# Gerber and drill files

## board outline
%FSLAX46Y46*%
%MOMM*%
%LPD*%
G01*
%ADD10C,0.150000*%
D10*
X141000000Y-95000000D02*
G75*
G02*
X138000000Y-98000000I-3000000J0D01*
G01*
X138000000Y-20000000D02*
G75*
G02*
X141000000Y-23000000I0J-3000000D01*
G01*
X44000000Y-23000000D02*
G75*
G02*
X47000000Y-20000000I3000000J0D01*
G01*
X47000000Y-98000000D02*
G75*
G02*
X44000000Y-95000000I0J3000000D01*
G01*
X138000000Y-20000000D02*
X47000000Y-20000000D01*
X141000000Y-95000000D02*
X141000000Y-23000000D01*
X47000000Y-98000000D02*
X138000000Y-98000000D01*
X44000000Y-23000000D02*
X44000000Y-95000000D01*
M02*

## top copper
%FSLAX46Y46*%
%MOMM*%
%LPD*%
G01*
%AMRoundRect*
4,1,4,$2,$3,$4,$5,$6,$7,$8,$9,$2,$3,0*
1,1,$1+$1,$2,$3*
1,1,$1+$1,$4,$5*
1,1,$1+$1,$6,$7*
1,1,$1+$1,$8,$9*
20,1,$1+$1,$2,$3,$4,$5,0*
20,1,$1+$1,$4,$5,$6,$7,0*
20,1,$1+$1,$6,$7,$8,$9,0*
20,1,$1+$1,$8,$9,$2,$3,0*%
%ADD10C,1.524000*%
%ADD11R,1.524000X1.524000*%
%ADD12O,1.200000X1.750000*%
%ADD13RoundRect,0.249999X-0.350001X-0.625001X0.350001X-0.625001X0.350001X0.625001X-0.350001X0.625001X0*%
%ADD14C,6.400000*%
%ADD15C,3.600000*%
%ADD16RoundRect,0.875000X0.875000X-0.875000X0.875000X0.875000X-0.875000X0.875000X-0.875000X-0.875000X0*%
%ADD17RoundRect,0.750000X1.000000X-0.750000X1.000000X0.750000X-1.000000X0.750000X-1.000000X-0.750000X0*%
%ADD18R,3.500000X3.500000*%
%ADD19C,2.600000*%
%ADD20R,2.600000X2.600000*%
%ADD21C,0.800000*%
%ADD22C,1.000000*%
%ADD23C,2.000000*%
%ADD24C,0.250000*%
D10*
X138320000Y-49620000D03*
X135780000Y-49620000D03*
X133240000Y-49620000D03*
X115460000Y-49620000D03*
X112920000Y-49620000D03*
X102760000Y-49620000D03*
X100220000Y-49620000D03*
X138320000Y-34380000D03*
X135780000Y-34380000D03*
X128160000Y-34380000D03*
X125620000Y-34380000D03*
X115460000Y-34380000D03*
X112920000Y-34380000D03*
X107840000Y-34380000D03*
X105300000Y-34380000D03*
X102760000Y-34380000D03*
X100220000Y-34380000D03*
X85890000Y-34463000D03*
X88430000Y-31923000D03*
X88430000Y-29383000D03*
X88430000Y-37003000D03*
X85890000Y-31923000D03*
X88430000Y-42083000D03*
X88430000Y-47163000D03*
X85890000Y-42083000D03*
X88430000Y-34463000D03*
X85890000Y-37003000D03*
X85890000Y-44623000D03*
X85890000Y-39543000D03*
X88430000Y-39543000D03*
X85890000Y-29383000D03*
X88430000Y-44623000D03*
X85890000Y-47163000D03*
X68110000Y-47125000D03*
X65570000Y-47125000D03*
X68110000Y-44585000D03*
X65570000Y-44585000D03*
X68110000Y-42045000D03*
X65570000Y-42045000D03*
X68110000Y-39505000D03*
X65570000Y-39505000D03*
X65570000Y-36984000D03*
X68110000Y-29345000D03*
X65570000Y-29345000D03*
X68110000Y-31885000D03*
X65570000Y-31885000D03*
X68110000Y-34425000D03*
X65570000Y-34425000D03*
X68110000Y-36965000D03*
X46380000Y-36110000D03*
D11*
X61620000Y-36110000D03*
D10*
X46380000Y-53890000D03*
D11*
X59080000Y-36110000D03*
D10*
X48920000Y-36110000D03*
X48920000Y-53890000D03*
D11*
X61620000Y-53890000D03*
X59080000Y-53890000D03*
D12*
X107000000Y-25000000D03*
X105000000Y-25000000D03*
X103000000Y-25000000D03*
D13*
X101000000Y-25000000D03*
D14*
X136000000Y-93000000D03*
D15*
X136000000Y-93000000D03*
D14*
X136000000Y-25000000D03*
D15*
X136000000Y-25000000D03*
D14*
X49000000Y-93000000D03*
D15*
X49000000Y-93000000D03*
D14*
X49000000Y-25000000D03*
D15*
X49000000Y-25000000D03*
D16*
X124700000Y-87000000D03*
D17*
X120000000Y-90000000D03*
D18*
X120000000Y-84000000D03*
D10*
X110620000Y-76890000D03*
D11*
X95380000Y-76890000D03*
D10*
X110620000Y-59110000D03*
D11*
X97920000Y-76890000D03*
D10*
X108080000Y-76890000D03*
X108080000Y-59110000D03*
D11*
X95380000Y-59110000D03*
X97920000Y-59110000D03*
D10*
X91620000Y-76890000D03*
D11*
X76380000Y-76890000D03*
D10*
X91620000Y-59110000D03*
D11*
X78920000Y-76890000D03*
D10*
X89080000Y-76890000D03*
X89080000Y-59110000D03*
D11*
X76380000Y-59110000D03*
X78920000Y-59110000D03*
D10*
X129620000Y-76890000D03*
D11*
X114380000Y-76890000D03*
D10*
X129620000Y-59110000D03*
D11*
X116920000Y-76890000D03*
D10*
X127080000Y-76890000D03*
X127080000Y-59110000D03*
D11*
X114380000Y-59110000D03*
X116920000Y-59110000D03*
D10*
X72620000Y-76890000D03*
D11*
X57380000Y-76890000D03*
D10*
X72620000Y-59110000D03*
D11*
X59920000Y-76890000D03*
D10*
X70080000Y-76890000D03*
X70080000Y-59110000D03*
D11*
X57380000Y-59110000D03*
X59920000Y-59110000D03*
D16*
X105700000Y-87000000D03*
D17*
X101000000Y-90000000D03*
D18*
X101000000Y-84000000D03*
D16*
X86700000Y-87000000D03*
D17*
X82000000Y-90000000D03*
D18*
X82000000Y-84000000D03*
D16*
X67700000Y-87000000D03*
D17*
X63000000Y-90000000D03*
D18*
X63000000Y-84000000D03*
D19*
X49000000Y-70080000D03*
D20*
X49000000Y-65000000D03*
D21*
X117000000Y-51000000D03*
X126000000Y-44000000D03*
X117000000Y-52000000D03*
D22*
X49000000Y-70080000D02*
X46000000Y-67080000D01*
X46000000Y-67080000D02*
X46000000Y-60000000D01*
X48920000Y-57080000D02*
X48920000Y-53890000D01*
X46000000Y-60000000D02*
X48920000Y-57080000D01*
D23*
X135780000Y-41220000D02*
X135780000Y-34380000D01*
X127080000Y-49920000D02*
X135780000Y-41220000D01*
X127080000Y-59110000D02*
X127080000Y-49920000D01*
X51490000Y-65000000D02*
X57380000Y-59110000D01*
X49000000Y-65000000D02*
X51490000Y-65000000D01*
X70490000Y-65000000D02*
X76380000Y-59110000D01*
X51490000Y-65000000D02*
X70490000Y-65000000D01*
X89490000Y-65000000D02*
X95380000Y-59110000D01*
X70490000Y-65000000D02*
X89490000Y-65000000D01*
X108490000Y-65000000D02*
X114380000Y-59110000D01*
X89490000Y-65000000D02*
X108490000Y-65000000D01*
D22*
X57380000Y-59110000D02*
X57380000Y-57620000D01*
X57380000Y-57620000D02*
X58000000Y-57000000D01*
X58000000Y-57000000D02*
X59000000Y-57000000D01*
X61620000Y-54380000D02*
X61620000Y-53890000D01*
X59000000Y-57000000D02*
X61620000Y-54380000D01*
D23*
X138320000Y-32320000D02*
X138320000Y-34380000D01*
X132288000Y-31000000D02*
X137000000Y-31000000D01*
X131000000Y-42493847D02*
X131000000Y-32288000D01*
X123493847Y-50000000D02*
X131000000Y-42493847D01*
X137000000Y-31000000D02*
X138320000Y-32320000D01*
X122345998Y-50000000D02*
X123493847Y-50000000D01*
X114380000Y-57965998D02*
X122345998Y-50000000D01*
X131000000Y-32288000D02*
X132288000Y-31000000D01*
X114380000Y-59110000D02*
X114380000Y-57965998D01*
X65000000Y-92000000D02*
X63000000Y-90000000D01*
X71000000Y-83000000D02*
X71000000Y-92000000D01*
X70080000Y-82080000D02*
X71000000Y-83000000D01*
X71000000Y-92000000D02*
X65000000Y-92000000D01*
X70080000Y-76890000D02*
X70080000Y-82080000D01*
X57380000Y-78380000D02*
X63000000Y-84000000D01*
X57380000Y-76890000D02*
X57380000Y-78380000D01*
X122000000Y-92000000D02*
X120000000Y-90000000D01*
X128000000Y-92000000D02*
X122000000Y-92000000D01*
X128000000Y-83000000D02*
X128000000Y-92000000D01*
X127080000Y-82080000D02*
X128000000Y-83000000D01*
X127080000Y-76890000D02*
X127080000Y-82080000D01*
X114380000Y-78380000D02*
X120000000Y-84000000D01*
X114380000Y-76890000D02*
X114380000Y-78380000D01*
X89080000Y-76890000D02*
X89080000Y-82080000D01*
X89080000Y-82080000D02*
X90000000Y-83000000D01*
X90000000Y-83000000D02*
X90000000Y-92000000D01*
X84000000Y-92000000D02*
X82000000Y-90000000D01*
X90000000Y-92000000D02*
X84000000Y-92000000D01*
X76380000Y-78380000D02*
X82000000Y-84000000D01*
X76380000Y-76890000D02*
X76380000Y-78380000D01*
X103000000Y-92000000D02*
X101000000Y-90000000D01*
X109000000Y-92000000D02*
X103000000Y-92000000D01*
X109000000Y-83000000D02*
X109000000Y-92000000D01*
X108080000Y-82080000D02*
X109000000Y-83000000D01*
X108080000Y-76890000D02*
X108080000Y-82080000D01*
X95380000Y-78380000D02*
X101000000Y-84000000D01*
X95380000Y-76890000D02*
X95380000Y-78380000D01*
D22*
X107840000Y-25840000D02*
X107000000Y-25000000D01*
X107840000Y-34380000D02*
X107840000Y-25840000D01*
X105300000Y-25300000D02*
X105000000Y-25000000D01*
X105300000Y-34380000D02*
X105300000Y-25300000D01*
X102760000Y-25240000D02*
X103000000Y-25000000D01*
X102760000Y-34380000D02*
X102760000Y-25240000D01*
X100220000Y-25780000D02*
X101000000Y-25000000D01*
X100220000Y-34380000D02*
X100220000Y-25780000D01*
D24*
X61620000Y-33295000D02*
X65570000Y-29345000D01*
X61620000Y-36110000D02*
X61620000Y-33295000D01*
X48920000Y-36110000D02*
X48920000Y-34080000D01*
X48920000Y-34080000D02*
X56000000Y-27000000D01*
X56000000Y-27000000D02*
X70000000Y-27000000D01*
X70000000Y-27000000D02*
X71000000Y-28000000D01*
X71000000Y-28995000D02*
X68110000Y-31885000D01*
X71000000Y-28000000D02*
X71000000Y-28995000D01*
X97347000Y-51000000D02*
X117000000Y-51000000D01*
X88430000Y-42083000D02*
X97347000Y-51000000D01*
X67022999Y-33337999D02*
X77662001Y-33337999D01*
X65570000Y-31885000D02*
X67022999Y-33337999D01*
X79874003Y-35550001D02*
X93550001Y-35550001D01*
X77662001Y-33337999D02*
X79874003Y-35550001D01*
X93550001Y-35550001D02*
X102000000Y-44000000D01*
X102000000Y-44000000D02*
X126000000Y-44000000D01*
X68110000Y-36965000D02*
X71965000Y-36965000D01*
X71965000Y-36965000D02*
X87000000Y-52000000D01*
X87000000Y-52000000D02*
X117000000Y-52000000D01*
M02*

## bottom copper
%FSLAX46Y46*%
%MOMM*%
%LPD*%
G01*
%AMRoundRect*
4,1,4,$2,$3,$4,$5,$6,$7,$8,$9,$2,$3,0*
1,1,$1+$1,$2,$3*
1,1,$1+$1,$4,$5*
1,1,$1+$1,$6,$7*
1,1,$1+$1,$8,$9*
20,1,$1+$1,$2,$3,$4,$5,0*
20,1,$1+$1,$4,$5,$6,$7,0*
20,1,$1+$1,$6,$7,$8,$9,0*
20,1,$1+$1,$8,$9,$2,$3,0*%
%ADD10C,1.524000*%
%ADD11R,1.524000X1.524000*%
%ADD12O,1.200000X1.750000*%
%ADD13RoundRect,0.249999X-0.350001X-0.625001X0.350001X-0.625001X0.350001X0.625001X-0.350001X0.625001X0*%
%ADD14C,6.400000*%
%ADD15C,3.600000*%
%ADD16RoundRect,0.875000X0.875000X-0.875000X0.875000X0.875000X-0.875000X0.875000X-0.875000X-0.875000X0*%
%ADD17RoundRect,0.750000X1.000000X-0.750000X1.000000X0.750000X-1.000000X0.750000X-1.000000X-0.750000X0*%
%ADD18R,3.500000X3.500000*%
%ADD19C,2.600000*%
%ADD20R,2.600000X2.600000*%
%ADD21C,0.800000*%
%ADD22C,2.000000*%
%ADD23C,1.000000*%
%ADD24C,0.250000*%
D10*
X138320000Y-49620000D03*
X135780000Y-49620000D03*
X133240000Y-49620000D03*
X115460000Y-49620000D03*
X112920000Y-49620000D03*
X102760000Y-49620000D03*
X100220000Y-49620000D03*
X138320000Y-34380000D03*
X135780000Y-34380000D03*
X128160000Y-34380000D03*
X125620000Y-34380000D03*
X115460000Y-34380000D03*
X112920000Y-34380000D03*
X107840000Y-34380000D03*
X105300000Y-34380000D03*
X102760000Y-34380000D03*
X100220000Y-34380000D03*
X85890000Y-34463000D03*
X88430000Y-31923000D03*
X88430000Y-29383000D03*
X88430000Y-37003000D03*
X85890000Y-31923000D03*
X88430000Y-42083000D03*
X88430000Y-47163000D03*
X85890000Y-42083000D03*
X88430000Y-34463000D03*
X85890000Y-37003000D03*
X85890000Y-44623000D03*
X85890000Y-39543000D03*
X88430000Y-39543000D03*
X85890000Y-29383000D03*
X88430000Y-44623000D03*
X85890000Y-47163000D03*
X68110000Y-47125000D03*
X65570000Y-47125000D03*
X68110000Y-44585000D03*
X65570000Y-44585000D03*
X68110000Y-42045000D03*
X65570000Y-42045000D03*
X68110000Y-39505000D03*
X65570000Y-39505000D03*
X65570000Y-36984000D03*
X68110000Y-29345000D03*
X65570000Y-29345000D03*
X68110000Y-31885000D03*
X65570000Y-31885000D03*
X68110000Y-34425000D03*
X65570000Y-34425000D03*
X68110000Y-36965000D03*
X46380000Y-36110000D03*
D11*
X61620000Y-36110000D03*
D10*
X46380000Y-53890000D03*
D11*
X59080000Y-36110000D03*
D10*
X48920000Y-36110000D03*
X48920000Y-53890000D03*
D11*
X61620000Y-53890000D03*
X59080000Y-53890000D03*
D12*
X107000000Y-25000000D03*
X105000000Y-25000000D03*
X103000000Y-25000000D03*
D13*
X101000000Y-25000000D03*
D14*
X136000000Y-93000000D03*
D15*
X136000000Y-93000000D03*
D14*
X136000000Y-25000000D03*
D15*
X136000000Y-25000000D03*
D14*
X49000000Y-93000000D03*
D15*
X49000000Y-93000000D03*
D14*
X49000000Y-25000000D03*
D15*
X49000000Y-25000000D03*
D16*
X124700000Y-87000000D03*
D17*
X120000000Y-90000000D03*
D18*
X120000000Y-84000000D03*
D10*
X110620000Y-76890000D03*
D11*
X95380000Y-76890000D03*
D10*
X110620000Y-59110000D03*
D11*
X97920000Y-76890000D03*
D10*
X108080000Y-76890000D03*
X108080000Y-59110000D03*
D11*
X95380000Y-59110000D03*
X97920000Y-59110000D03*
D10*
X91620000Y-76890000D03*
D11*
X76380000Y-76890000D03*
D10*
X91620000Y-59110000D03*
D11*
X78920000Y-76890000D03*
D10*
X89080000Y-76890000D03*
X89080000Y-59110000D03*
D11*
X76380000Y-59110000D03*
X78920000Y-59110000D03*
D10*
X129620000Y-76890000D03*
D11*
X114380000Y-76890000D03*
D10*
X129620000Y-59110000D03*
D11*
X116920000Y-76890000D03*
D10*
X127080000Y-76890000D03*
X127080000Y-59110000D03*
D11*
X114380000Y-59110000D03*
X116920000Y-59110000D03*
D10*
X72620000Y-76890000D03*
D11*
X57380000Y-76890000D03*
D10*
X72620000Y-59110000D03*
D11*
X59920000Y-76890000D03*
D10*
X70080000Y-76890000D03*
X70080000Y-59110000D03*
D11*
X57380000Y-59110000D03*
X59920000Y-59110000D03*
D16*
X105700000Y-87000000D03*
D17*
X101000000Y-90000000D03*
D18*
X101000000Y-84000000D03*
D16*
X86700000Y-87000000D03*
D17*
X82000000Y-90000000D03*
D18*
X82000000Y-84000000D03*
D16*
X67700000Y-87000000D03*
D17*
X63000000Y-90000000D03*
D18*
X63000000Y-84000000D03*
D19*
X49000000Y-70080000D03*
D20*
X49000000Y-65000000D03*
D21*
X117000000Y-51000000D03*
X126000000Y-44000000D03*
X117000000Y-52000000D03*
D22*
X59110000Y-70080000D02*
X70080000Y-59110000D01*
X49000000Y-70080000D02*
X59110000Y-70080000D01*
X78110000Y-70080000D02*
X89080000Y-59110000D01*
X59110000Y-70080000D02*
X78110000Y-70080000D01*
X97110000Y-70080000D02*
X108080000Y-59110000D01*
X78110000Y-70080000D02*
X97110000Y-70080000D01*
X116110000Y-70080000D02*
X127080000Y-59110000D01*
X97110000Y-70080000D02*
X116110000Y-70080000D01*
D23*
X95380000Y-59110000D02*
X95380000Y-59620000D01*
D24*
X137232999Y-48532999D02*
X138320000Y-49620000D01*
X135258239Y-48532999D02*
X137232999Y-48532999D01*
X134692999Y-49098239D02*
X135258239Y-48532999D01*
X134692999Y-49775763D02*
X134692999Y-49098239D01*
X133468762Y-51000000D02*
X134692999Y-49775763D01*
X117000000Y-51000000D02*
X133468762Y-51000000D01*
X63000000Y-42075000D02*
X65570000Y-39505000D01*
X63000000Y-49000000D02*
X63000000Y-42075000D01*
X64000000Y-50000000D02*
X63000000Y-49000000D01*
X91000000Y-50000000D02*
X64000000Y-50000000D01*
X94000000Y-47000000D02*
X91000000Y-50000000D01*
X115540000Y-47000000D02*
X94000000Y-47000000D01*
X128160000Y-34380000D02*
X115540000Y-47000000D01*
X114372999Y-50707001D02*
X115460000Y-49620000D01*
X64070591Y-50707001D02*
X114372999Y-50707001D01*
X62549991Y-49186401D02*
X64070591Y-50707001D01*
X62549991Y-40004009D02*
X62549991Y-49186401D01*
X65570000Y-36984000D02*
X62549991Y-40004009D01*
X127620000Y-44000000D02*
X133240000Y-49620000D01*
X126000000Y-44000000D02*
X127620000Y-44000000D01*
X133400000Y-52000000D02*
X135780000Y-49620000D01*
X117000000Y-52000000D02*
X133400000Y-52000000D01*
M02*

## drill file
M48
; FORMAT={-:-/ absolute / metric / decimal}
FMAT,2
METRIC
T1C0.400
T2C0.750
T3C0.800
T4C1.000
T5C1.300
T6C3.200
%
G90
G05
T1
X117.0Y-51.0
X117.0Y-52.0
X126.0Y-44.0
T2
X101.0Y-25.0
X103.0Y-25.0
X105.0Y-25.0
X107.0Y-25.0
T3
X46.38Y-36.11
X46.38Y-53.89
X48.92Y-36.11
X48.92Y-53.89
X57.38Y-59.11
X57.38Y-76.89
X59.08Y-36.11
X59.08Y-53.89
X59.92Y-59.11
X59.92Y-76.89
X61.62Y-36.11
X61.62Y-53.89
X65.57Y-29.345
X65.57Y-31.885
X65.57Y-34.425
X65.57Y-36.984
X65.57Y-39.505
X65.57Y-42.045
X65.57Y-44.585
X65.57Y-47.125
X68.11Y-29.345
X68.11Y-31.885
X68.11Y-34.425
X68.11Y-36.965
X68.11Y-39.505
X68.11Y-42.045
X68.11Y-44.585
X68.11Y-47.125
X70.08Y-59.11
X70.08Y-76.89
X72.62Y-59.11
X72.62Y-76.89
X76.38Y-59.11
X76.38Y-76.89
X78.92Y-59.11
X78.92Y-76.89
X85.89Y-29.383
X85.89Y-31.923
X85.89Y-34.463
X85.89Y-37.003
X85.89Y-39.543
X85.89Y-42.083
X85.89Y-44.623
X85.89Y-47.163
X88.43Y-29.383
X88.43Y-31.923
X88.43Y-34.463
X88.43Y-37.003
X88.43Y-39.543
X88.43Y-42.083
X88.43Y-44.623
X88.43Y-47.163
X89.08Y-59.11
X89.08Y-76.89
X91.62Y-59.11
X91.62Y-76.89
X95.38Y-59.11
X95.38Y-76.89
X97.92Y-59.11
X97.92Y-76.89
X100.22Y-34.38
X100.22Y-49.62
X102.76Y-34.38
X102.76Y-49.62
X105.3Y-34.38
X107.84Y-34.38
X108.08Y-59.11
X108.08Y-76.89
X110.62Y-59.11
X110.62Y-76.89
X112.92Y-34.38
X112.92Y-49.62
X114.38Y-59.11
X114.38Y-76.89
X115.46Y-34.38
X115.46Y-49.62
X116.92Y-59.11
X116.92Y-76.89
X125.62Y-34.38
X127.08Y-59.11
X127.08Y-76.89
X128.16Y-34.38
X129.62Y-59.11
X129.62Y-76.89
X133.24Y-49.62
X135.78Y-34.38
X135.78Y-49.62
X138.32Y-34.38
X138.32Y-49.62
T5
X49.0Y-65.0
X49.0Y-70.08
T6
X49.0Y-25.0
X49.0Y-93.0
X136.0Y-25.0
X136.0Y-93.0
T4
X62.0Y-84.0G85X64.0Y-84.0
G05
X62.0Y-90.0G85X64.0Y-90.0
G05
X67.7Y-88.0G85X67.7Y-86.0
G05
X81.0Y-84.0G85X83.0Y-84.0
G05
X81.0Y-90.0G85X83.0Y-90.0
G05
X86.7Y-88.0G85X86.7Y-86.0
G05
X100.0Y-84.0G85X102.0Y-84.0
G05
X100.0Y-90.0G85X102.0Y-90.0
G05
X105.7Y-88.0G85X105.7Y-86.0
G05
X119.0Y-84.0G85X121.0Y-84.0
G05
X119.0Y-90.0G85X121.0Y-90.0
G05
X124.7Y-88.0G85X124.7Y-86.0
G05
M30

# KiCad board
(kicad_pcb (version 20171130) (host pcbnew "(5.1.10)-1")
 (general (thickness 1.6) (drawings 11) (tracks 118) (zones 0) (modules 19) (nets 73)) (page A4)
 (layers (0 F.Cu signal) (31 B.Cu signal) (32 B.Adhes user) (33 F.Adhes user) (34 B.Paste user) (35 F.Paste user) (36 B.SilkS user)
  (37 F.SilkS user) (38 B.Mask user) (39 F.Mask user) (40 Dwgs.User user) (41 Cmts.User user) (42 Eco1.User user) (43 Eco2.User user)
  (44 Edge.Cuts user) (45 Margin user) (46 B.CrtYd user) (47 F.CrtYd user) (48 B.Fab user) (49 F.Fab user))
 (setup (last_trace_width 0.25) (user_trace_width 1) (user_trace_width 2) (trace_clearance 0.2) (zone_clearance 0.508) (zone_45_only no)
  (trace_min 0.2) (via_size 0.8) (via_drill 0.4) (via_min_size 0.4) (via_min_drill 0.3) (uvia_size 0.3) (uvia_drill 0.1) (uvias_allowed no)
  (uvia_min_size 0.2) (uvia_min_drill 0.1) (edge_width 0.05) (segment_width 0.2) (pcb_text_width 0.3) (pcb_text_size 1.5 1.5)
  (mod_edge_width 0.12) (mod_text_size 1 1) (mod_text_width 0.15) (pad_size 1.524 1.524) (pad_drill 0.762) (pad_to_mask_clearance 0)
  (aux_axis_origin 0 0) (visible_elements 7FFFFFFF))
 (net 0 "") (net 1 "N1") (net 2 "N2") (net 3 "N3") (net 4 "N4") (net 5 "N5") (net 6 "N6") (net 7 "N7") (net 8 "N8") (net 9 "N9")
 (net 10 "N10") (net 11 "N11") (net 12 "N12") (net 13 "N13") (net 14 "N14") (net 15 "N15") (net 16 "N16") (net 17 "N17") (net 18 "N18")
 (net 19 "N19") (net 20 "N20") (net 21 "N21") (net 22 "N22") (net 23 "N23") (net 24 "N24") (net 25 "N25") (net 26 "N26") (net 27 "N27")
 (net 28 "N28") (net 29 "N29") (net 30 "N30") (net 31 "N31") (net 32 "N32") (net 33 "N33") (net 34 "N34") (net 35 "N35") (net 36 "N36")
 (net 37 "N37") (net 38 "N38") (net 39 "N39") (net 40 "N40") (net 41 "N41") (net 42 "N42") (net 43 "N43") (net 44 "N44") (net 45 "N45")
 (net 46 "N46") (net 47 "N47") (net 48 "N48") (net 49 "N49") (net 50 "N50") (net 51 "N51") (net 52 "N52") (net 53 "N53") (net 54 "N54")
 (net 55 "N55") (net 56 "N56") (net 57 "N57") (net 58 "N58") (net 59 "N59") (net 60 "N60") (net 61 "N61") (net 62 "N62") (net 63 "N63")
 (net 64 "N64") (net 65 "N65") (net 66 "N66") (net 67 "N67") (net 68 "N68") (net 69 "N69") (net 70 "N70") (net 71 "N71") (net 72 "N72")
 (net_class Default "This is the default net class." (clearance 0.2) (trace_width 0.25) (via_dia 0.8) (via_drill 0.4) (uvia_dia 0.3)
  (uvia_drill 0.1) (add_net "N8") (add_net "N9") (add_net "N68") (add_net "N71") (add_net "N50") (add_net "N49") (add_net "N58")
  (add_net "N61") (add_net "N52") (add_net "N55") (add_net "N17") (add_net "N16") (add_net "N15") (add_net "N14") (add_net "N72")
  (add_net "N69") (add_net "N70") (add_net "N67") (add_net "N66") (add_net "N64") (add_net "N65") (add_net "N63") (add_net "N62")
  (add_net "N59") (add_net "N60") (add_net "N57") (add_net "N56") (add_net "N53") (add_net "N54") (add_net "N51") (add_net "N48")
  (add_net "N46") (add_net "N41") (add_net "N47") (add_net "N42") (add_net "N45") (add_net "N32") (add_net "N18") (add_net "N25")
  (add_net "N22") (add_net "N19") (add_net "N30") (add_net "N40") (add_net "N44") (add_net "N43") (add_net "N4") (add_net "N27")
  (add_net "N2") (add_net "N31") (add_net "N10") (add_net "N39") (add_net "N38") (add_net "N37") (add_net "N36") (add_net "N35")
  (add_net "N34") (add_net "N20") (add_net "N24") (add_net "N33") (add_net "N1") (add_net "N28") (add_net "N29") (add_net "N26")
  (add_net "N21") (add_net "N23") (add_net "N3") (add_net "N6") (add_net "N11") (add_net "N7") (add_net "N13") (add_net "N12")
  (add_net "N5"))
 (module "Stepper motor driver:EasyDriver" (layer F.Cu) (at 118 42)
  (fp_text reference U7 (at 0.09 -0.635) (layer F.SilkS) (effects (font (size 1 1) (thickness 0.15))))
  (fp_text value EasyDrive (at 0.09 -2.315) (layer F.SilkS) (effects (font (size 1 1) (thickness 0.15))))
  (pad DIR thru_hole circle (at 20.32 7.62) (size 1.524 1.524) (drill 0.8) (layers *.Cu *.Mask) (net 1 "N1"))
  (pad STP thru_hole circle (at 17.78 7.62) (size 1.524 1.524) (drill 0.8) (layers *.Cu *.Mask) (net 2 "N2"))
  (pad GND thru_hole circle (at 15.24 7.62 270) (size 1.524 1.524) (drill 0.8) (layers *.Cu *.Mask) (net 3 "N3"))
  (pad MS1 thru_hole circle (at -2.54 7.62) (size 1.524 1.524) (drill 0.8) (layers *.Cu *.Mask) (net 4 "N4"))
  (pad SLP thru_hole circle (at -5.08 7.62) (size 1.524 1.524) (drill 0.8) (layers *.Cu *.Mask) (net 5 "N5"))
  (pad 5V+ thru_hole circle (at -15.24 7.62) (size 1.524 1.524) (drill 0.8) (layers *.Cu *.Mask) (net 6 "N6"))
  (pad GND_alt thru_hole circle (at -17.78 7.62) (size 1.524 1.524) (drill 0.8) (layers *.Cu *.Mask) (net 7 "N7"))
  (pad M+ thru_hole circle (at 20.32 -7.62) (size 1.524 1.524) (drill 0.8) (layers *.Cu *.Mask) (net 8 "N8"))
  (pad GND_IN thru_hole circle (at 17.78 -7.62) (size 1.524 1.524) (drill 0.8) (layers *.Cu *.Mask) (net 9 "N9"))
  (pad MS2 thru_hole circle (at 10.16 -7.62) (size 1.524 1.524) (drill 0.8) (layers *.Cu *.Mask) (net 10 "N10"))
  (pad EN thru_hole circle (at 7.62 -7.62) (size 1.524 1.524) (drill 0.8) (layers *.Cu *.Mask) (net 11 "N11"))
  (pad RST thru_hole circle (at -2.54 -7.62) (size 1.524 1.524) (drill 0.8) (layers *.Cu *.Mask) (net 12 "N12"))
  (pad PFD thru_hole circle (at -5.08 -7.62) (size 1.524 1.524) (drill 0.8) (layers *.Cu *.Mask) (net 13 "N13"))
  (pad B- thru_hole circle (at -10.16 -7.62) (size 1.524 1.524) (drill 0.8) (layers *.Cu *.Mask) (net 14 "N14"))
  (pad B+ thru_hole circle (at -12.7 -7.62) (size 1.524 1.524) (drill 0.8) (layers *.Cu *.Mask) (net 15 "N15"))
  (pad A- thru_hole circle (at -15.24 -7.62) (size 1.524 1.524) (drill 0.8) (layers *.Cu *.Mask) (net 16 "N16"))
  (pad A+ thru_hole circle (at -17.78 -7.62) (size 1.524 1.524) (drill 0.8) (layers *.Cu *.Mask) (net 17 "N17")))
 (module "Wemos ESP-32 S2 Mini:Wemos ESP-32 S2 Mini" (layer F.Cu) (at 77 38 270)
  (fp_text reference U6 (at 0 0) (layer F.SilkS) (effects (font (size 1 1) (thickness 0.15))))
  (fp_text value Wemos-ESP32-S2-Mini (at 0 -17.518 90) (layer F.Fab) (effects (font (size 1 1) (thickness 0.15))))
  (pad 10 thru_hole circle (at -3.537 -8.89 270) (size 1.524 1.524) (drill 0.8) (layers *.Cu *.Mask) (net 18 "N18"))
  (pad 13 thru_hole circle (at -6.077 -11.43 270) (size 1.524 1.524) (drill 0.8) (layers *.Cu *.Mask) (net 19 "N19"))
  (pad 3V3 thru_hole circle (at -8.617 -11.43 270) (size 1.524 1.524) (drill 0.8) (layers *.Cu *.Mask) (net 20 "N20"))
  (pad 9 thru_hole circle (at -0.997 -11.43 270) (size 1.524 1.524) (drill 0.8) (layers *.Cu *.Mask) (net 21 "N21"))
  (pad 12 thru_hole circle (at -6.077 -8.89 270) (size 1.524 1.524) (drill 0.8) (layers *.Cu *.Mask) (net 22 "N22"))
  (pad 5 thru_hole circle (at 4.083 -11.43 270) (size 1.524 1.524) (drill 0.8) (layers *.Cu *.Mask) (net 1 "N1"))
  (pad EN thru_hole circle (at 9.163 -11.43 270) (size 1.524 1.524) (drill 0.8) (layers *.Cu *.Mask) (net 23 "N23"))
  (pad 4 thru_hole circle (at 4.083 -8.89 270) (size 1.524 1.524) (drill 0.8) (layers *.Cu *.Mask) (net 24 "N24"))
  (pad 11 thru_hole circle (at -3.537 -11.43 270) (size 1.524 1.524) (drill 0.8) (layers *.Cu *.Mask) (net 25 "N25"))
  (pad 8 thru_hole circle (at -0.997 -8.89 270) (size 1.524 1.524) (drill 0.8) (layers *.Cu *.Mask) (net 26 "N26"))
  (pad 2 thru_hole circle (at 6.623 -8.89 270) (size 1.524 1.524) (drill 0.8) (layers *.Cu *.Mask) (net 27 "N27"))
  (pad 6 thru_hole circle (at 1.543 -8.89 270) (size 1.524 1.524) (drill 0.8) (layers *.Cu *.Mask) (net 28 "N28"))
  (pad 7 thru_hole circle (at 1.543 -11.43 270) (size 1.524 1.524) (drill 0.8) (layers *.Cu *.Mask) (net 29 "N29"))
  (pad 14 thru_hole circle (at -8.617 -8.89 270) (size 1.524 1.524) (drill 0.8) (layers *.Cu *.Mask) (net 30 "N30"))
  (pad 3 thru_hole circle (at 6.623 -11.43 270) (size 1.524 1.524) (drill 0.8) (layers *.Cu *.Mask) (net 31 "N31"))
  (pad 1 thru_hole circle (at 9.163 -8.89 270) (size 1.524 1.524) (drill 0.8) (layers *.Cu *.Mask) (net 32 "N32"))
  (pad 40 thru_hole circle (at 9.125 8.89 270) (size 1.524 1.524) (drill 0.8) (layers *.Cu *.Mask) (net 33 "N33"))
  (pad 39 thru_hole circle (at 9.125 11.43 270) (size 1.524 1.524) (drill 0.8) (layers *.Cu *.Mask) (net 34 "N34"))
  (pad 38 thru_hole circle (at 6.585 8.89 270) (size 1.524 1.524) (drill 0.8) (layers *.Cu *.Mask) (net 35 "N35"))
  (pad 37 thru_hole circle (at 6.585 11.43 270) (size 1.524 1.524) (drill 0.8) (layers *.Cu *.Mask) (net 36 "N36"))
  (pad 36 thru_hole circle (at 4.045 8.89 270) (size 1.524 1.524) (drill 0.8) (layers *.Cu *.Mask) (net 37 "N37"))
  (pad 35 thru_hole circle (at 4.045 11.43 270) (size 1.524 1.524) (drill 0.8) (layers *.Cu *.Mask) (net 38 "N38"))
  (pad 34 thru_hole circle (at 1.505 8.89 270) (size 1.524 1.524) (drill 0.8) (layers *.Cu *.Mask) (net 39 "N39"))
  (pad 33 thru_hole circle (at 1.505 11.43 270) (size 1.524 1.524) (drill 0.8) (layers *.Cu *.Mask) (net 10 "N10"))
  (pad 18 thru_hole circle (at -1.016 11.43 270) (size 1.524 1.524) (drill 0.8) (layers *.Cu *.Mask) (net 4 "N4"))
  (pad 15 thru_hole circle (at -8.655 8.89 270) (size 1.524 1.524) (drill 0.8) (layers *.Cu *.Mask) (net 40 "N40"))
  (pad VBUS thru_hole circle (at -8.655 11.43 270) (size 1.524 1.524) (drill 0.8) (layers *.Cu *.Mask) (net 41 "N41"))
  (pad GND_INNER thru_hole circle (at -6.115 8.89 270) (size 1.524 1.524) (drill 0.8) (layers *.Cu *.Mask) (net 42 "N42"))
  (pad GND_OUTER thru_hole circle (at -6.115 11.43 270) (size 1.524 1.524) (drill 0.8) (layers *.Cu *.Mask) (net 3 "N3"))
  (pad 17 thru_hole circle (at -3.575 8.89 270) (size 1.524 1.524) (drill 0.8) (layers *.Cu *.Mask) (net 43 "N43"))
  (pad 16 thru_hole circle (at -3.575 11.43 270) (size 1.524 1.524) (drill 0.8) (layers *.Cu *.Mask) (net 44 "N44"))
  (pad 21 thru_hole circle (at -1.035 8.89 270) (size 1.524 1.524) (drill 0.8) (layers *.Cu *.Mask) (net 2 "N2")))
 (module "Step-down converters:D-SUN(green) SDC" (layer F.Cu) (at 54 45 180)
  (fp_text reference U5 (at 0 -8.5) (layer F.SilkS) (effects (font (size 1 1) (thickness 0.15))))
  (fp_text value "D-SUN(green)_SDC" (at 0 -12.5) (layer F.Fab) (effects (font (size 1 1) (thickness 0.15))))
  (pad 8 thru_hole circle (at 7.62 8.89 180) (size 1.524 1.524) (drill 0.8) (layers *.Cu *.Mask) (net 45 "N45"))
  (pad 5 thru_hole rect (at -7.62 8.89 180) (size 1.524 1.524) (drill 0.8) (layers *.Cu *.Mask) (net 41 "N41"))
  (pad 4 thru_hole circle (at 7.62 -8.89 180) (size 1.524 1.524) (drill 0.8) (layers *.Cu *.Mask) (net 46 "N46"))
  (pad 6 thru_hole rect (at -5.08 8.89 180) (size 1.524 1.524) (drill 0.8) (layers *.Cu *.Mask) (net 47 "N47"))
  (pad 7 thru_hole circle (at 5.08 8.89 180) (size 1.524 1.524) (drill 0.8) (layers *.Cu *.Mask) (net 42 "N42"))
  (pad 3 thru_hole circle (at 5.08 -8.89 180) (size 1.524 1.524) (drill 0.8) (layers *.Cu *.Mask) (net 9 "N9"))
  (pad 1 thru_hole rect (at -7.62 -8.89 180) (size 1.524 1.524) (drill 0.8) (layers *.Cu *.Mask) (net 8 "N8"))
  (pad 2 thru_hole rect (at -5.08 -8.89 180) (size 1.524 1.524) (drill 0.8) (layers *.Cu *.Mask) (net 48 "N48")))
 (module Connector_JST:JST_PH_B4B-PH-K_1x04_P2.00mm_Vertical (layer F.Cu) (at 101 25)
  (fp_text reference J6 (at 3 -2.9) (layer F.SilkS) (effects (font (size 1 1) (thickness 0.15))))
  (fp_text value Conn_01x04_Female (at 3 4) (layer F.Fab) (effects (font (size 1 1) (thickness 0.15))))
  (pad 4 thru_hole oval (at 6 0) (size 1.2 1.75) (drill 0.75) (layers *.Cu *.Mask) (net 14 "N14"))
  (pad 3 thru_hole oval (at 4 0) (size 1.2 1.75) (drill 0.75) (layers *.Cu *.Mask) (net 15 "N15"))
  (pad 2 thru_hole oval (at 2 0) (size 1.2 1.75) (drill 0.75) (layers *.Cu *.Mask) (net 16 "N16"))
  (pad 1 thru_hole roundrect (at 0 0) (size 1.2 1.75) (drill 0.75) (layers *.Cu *.Mask) (roundrect_rratio 0.2083325) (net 17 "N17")))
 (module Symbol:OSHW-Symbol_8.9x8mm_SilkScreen (layer F.Cu) (at 50 78)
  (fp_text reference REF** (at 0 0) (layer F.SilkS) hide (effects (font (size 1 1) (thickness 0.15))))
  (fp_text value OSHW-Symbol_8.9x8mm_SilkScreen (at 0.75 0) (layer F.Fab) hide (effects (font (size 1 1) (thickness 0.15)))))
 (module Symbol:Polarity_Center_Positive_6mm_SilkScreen (layer F.Cu) (at 136 75 270)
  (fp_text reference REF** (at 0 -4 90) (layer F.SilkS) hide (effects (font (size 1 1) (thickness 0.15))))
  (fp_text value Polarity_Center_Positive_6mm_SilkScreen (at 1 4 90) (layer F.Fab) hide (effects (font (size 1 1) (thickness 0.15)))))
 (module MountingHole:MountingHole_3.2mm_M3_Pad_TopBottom (layer F.Cu) (at 136 93)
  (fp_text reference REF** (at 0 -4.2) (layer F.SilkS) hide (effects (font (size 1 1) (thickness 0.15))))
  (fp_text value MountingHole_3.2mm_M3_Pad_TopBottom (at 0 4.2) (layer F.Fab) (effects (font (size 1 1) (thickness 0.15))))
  (pad 1 connect circle (at 0 0) (size 6.4 6.4) (layers B.Cu B.Mask))
  (pad 1 connect circle (at 0 0) (size 6.4 6.4) (layers F.Cu F.Mask))
  (pad 1 thru_hole circle (at 0 0) (size 3.6 3.6) (drill 3.2) (layers *.Cu *.Mask)))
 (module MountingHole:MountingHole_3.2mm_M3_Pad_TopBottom (layer F.Cu) (at 136 25)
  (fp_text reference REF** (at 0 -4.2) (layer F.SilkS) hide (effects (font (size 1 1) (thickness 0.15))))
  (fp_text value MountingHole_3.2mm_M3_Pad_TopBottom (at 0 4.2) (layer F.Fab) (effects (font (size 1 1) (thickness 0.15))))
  (pad 1 connect circle (at 0 0) (size 6.4 6.4) (layers B.Cu B.Mask))
  (pad 1 connect circle (at 0 0) (size 6.4 6.4) (layers F.Cu F.Mask))
  (pad 1 thru_hole circle (at 0 0) (size 3.6 3.6) (drill 3.2) (layers *.Cu *.Mask)))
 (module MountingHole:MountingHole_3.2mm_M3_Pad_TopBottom (layer F.Cu) (at 49 93)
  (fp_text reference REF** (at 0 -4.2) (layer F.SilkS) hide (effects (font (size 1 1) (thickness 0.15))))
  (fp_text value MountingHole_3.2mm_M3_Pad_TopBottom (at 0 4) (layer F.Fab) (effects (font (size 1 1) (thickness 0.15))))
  (pad 1 connect circle (at 0 0) (size 6.4 6.4) (layers B.Cu B.Mask))
  (pad 1 connect circle (at 0 0) (size 6.4 6.4) (layers F.Cu F.Mask))
  (pad 1 thru_hole circle (at 0 0) (size 3.6 3.6) (drill 3.2) (layers *.Cu *.Mask)))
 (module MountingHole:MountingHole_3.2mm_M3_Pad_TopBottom (layer F.Cu) (at 49 25)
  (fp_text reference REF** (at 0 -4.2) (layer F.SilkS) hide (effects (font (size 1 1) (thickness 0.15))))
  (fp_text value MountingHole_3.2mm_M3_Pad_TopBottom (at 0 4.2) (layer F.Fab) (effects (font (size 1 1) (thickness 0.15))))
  (pad 1 connect circle (at 0 0) (size 6.4 6.4) (layers B.Cu B.Mask))
  (pad 1 connect circle (at 0 0) (size 6.4 6.4) (layers F.Cu F.Mask))
  (pad 1 thru_hole circle (at 0 0) (size 3.6 3.6) (drill 3.2) (layers *.Cu *.Mask)))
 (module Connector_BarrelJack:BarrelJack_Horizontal (layer F.Cu) (at 120 84 90)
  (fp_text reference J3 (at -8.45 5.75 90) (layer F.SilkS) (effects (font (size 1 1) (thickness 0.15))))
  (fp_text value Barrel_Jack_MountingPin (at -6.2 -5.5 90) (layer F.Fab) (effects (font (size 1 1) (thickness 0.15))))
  (pad 3 thru_hole roundrect (at -3 4.7 90) (size 3.5 3.5) (drill oval 3 1) (layers *.Cu *.Mask) (roundrect_rratio 0.25))
  (pad 2 thru_hole roundrect (at -6 0 90) (size 3 3.5) (drill oval 1 3) (layers *.Cu *.Mask) (roundrect_rratio 0.25) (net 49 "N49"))
  (pad 1 thru_hole rect (at 0 0 90) (size 3.5 3.5) (drill oval 1 3) (layers *.Cu *.Mask) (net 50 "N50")))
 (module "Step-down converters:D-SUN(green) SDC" (layer F.Cu) (at 103 68)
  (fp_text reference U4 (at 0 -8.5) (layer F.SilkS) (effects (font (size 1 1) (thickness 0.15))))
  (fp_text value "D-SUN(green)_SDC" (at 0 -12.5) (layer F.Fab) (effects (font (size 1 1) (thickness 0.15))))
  (pad 8 thru_hole circle (at 7.62 8.89) (size 1.524 1.524) (drill 0.8) (layers *.Cu *.Mask) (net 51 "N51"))
  (pad 5 thru_hole rect (at -7.62 8.89) (size 1.524 1.524) (drill 0.8) (layers *.Cu *.Mask) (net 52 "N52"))
  (pad 4 thru_hole circle (at 7.62 -8.89) (size 1.524 1.524) (drill 0.8) (layers *.Cu *.Mask) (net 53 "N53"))
  (pad 6 thru_hole rect (at -5.08 8.89) (size 1.524 1.524) (drill 0.8) (layers *.Cu *.Mask) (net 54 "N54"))
  (pad 7 thru_hole circle (at 5.08 8.89) (size 1.524 1.524) (drill 0.8) (layers *.Cu *.Mask) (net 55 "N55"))
  (pad 3 thru_hole circle (at 5.08 -8.89) (size 1.524 1.524) (drill 0.8) (layers *.Cu *.Mask) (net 9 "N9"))
  (pad 1 thru_hole rect (at -7.62 -8.89) (size 1.524 1.524) (drill 0.8) (layers *.Cu *.Mask) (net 8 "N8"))
  (pad 2 thru_hole rect (at -5.08 -8.89) (size 1.524 1.524) (drill 0.8) (layers *.Cu *.Mask) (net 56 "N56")))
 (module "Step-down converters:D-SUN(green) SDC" (layer F.Cu) (at 84 68)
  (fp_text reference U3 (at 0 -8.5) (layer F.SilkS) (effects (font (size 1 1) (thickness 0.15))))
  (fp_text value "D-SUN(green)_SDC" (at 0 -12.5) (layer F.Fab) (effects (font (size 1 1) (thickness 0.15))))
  (pad 8 thru_hole circle (at 7.62 8.89) (size 1.524 1.524) (drill 0.8) (layers *.Cu *.Mask) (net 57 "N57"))
  (pad 5 thru_hole rect (at -7.62 8.89) (size 1.524 1.524) (drill 0.8) (layers *.Cu *.Mask) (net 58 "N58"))
  (pad 4 thru_hole circle (at 7.62 -8.89) (size 1.524 1.524) (drill 0.8) (layers *.Cu *.Mask) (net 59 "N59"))
  (pad 6 thru_hole rect (at -5.08 8.89) (size 1.524 1.524) (drill 0.8) (layers *.Cu *.Mask) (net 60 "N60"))
  (pad 7 thru_hole circle (at 5.08 8.89) (size 1.524 1.524) (drill 0.8) (layers *.Cu *.Mask) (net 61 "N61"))
  (pad 3 thru_hole circle (at 5.08 -8.89) (size 1.524 1.524) (drill 0.8) (layers *.Cu *.Mask) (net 9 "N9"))
  (pad 1 thru_hole rect (at -7.62 -8.89) (size 1.524 1.524) (drill 0.8) (layers *.Cu *.Mask) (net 8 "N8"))
  (pad 2 thru_hole rect (at -5.08 -8.89) (size 1.524 1.524) (drill 0.8) (layers *.Cu *.Mask) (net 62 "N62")))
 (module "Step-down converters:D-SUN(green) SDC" (layer F.Cu) (at 122 68)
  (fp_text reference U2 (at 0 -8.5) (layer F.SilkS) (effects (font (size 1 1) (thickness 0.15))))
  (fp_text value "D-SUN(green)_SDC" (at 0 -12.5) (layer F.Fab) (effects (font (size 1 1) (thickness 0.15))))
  (pad 8 thru_hole circle (at 7.62 8.89) (size 1.524 1.524) (drill 0.8) (layers *.Cu *.Mask) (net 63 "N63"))
  (pad 5 thru_hole rect (at -7.62 8.89) (size 1.524 1.524) (drill 0.8) (layers *.Cu *.Mask) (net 50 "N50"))
  (pad 4 thru_hole circle (at 7.62 -8.89) (size 1.524 1.524) (drill 0.8) (layers *.Cu *.Mask) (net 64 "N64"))
  (pad 6 thru_hole rect (at -5.08 8.89) (size 1.524 1.524) (drill 0.8) (layers *.Cu *.Mask) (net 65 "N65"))
  (pad 7 thru_hole circle (at 5.08 8.89) (size 1.524 1.524) (drill 0.8) (layers *.Cu *.Mask) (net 49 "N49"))
  (pad 3 thru_hole circle (at 5.08 -8.89) (size 1.524 1.524) (drill 0.8) (layers *.Cu *.Mask) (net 9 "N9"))
  (pad 1 thru_hole rect (at -7.62 -8.89) (size 1.524 1.524) (drill 0.8) (layers *.Cu *.Mask) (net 8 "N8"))
  (pad 2 thru_hole rect (at -5.08 -8.89) (size 1.524 1.524) (drill 0.8) (layers *.Cu *.Mask) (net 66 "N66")))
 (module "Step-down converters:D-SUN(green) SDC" (layer F.Cu) (at 65 68)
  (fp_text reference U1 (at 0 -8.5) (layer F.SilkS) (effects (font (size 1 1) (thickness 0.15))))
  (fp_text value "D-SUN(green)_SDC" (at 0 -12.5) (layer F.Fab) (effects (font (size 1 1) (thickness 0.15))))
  (pad 8 thru_hole circle (at 7.62 8.89) (size 1.524 1.524) (drill 0.8) (layers *.Cu *.Mask) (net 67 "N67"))
  (pad 5 thru_hole rect (at -7.62 8.89) (size 1.524 1.524) (drill 0.8) (layers *.Cu *.Mask) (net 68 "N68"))
  (pad 4 thru_hole circle (at 7.62 -8.89) (size 1.524 1.524) (drill 0.8) (layers *.Cu *.Mask) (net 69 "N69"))
  (pad 6 thru_hole rect (at -5.08 8.89) (size 1.524 1.524) (drill 0.8) (layers *.Cu *.Mask) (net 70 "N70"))
  (pad 7 thru_hole circle (at 5.08 8.89) (size 1.524 1.524) (drill 0.8) (layers *.Cu *.Mask) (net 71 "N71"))
  (pad 3 thru_hole circle (at 5.08 -8.89) (size 1.524 1.524) (drill 0.8) (layers *.Cu *.Mask) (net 9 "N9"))
  (pad 1 thru_hole rect (at -7.62 -8.89) (size 1.524 1.524) (drill 0.8) (layers *.Cu *.Mask) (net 8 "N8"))
  (pad 2 thru_hole rect (at -5.08 -8.89) (size 1.524 1.524) (drill 0.8) (layers *.Cu *.Mask) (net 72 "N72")))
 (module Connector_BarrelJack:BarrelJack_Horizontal (layer F.Cu) (at 101 84 90)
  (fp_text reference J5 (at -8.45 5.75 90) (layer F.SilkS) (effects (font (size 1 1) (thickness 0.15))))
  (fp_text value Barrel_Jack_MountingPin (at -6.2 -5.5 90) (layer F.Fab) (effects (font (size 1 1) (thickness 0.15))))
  (pad 3 thru_hole roundrect (at -3 4.7 90) (size 3.5 3.5) (drill oval 3 1) (layers *.Cu *.Mask) (roundrect_rratio 0.25))
  (pad 2 thru_hole roundrect (at -6 0 90) (size 3 3.5) (drill oval 1 3) (layers *.Cu *.Mask) (roundrect_rratio 0.25) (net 55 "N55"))
  (pad 1 thru_hole rect (at 0 0 90) (size 3.5 3.5) (drill oval 1 3) (layers *.Cu *.Mask) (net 52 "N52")))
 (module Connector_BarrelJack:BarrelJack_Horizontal (layer F.Cu) (at 82 84 90)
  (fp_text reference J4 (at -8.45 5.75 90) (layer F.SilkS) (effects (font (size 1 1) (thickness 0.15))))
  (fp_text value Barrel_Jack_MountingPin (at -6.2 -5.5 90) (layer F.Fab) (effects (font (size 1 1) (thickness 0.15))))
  (pad 3 thru_hole roundrect (at -3 4.7 90) (size 3.5 3.5) (drill oval 3 1) (layers *.Cu *.Mask) (roundrect_rratio 0.25))
  (pad 2 thru_hole roundrect (at -6 0 90) (size 3 3.5) (drill oval 1 3) (layers *.Cu *.Mask) (roundrect_rratio 0.25) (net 61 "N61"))
  (pad 1 thru_hole rect (at 0 0 90) (size 3.5 3.5) (drill oval 1 3) (layers *.Cu *.Mask) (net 58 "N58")))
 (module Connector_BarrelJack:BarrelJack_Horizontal (layer F.Cu) (at 63 84 90)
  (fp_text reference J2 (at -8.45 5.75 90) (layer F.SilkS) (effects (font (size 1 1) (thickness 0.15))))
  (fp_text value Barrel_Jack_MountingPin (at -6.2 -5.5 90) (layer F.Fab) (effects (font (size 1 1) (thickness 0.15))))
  (pad 3 thru_hole roundrect (at -3 4.7 90) (size 3.5 3.5) (drill oval 3 1) (layers *.Cu *.Mask) (roundrect_rratio 0.25))
  (pad 2 thru_hole roundrect (at -6 0 90) (size 3 3.5) (drill oval 1 3) (layers *.Cu *.Mask) (roundrect_rratio 0.25) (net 71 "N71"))
  (pad 1 thru_hole rect (at 0 0 90) (size 3.5 3.5) (drill oval 1 3) (layers *.Cu *.Mask) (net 68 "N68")))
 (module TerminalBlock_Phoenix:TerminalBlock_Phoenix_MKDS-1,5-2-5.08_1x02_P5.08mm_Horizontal (layer F.Cu) (at 49 65 270)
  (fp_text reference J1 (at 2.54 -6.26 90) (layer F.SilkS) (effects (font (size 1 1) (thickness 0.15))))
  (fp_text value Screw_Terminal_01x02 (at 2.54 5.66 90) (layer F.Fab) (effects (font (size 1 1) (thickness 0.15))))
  (pad 2 thru_hole circle (at 5.08 0 270) (size 2.6 2.6) (drill 1.3) (layers *.Cu *.Mask) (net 9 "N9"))
  (pad 1 thru_hole rect (at 0 0 270) (size 2.6 2.6) (drill 1.3) (layers *.Cu *.Mask) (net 8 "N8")))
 (gr_arc (start 138 95) (end 138 98) (angle -90) (layer Edge.Cuts) (width 0.15))
 (gr_arc (start 138 23) (end 141 23) (angle -90) (layer Edge.Cuts) (width 0.15))
 (gr_arc (start 47 23) (end 47 20) (angle -90) (layer Edge.Cuts) (width 0.15))
 (gr_arc (start 47 95) (end 44 95) (angle -90) (layer Edge.Cuts) (width 0.15))
 (gr_line (start 138 20) (end 47 20) (layer Edge.Cuts) (width 0.15))
 (gr_line (start 141 95) (end 141 23) (layer Edge.Cuts) (width 0.15))
 (gr_line (start 47 98) (end 138 98) (layer Edge.Cuts) (width 0.15))
 (gr_line (start 44 23) (end 44 95) (layer Edge.Cuts) (width 0.15))
 (segment (start 59.11 70.08) (end 70.08 59.11) (width 2) (layer B.Cu) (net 9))
 (segment (start 49 70.08) (end 59.11 70.08) (width 2) (layer B.Cu) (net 9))
 (segment (start 78.11 70.08) (end 89.08 59.11) (width 2) (layer B.Cu) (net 9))
 (segment (start 59.11 70.08) (end 78.11 70.08) (width 2) (layer B.Cu) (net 9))
 (segment (start 97.11 70.08) (end 108.08 59.11) (width 2) (layer B.Cu) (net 9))
 (segment (start 78.11 70.08) (end 97.11 70.08) (width 2) (layer B.Cu) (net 9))
 (segment (start 116.11 70.08) (end 127.08 59.11) (width 2) (layer B.Cu) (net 9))
 (segment (start 97.11 70.08) (end 116.11 70.08) (width 2) (layer B.Cu) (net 9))
 (segment (start 49 70.08) (end 46 67.08) (width 1) (layer F.Cu) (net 9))
 (segment (start 46 67.08) (end 46 60) (width 1) (layer F.Cu) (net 9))
 (segment (start 48.92 57.08) (end 48.92 53.89) (width 1) (layer F.Cu) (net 9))
 (segment (start 46 60) (end 48.92 57.08) (width 1) (layer F.Cu) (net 9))
 (segment (start 135.78 41.22) (end 135.78 34.38) (width 2) (layer F.Cu) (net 9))
 (segment (start 127.08 49.92) (end 135.78 41.22) (width 2) (layer F.Cu) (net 9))
 (segment (start 127.08 59.11) (end 127.08 49.92) (width 2) (layer F.Cu) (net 9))
 (segment (start 95.38 59.11) (end 95.38 59.62) (width 1) (layer B.Cu) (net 8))
 (segment (start 51.49 65) (end 57.38 59.11) (width 2) (layer F.Cu) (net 8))
 (segment (start 49 65) (end 51.49 65) (width 2) (layer F.Cu) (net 8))
 (segment (start 70.49 65) (end 76.38 59.11) (width 2) (layer F.Cu) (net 8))
 (segment (start 51.49 65) (end 70.49 65) (width 2) (layer F.Cu) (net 8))
 (segment (start 89.49 65) (end 95.38 59.11) (width 2) (layer F.Cu) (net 8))
 (segment (start 70.49 65) (end 89.49 65) (width 2) (layer F.Cu) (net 8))
 (segment (start 108.49 65) (end 114.38 59.11) (width 2) (layer F.Cu) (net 8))
 (segment (start 89.49 65) (end 108.49 65) (width 2) (layer F.Cu) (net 8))
 (segment (start 57.38 59.11) (end 57.38 57.62) (width 1) (layer F.Cu) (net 8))
 (segment (start 57.38 57.62) (end 58 57) (width 1) (layer F.Cu) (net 8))
 (segment (start 58 57) (end 59 57) (width 1) (layer F.Cu) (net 8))
 (segment (start 61.62 54.38) (end 61.62 53.89) (width 1) (layer F.Cu) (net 8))
 (segment (start 59 57) (end 61.62 54.38) (width 1) (layer F.Cu) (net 8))
 (segment (start 138.32 32.32) (end 138.32 34.38) (width 2) (layer F.Cu) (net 8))
 (segment (start 132.288 31) (end 137 31) (width 2) (layer F.Cu) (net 8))
 (segment (start 131 42.493847) (end 131 32.288) (width 2) (layer F.Cu) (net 8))
 (segment (start 123.493847 50) (end 131 42.493847) (width 2) (layer F.Cu) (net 8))
 (segment (start 137 31) (end 138.32 32.32) (width 2) (layer F.Cu) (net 8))
 (segment (start 122.345998 50) (end 123.493847 50) (width 2) (layer F.Cu) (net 8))
 (segment (start 114.38 57.965998) (end 122.345998 50) (width 2) (layer F.Cu) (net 8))
 (segment (start 131 32.288) (end 132.288 31) (width 2) (layer F.Cu) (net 8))
 (segment (start 114.38 59.11) (end 114.38 57.965998) (width 2) (layer F.Cu) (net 8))
 (segment (start 65 92) (end 63 90) (width 2) (layer F.Cu) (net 71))
 (segment (start 71 83) (end 71 92) (width 2) (layer F.Cu) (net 71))
 (segment (start 70.08 82.08) (end 71 83) (width 2) (layer F.Cu) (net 71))
 (segment (start 71 92) (end 65 92) (width 2) (layer F.Cu) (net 71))
 (segment (start 70.08 76.89) (end 70.08 82.08) (width 2) (layer F.Cu) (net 71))
 (segment (start 57.38 78.38) (end 63 84) (width 2) (layer F.Cu) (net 68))
 (segment (start 57.38 76.89) (end 57.38 78.38) (width 2) (layer F.Cu) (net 68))
 (segment (start 122 92) (end 120 90) (width 2) (layer F.Cu) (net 49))
 (segment (start 128 92) (end 122 92) (width 2) (layer F.Cu) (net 49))
 (segment (start 128 83) (end 128 92) (width 2) (layer F.Cu) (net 49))
 (segment (start 127.08 82.08) (end 128 83) (width 2) (layer F.Cu) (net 49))
 (segment (start 127.08 76.89) (end 127.08 82.08) (width 2) (layer F.Cu) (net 49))
 (segment (start 114.38 78.38) (end 120 84) (width 2) (layer F.Cu) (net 50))
 (segment (start 114.38 76.89) (end 114.38 78.38) (width 2) (layer F.Cu) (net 50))
 (segment (start 89.08 76.89) (end 89.08 82.08) (width 2) (layer F.Cu) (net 61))
 (segment (start 89.08 82.08) (end 90 83) (width 2) (layer F.Cu) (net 61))
 (segment (start 90 83) (end 90 92) (width 2) (layer F.Cu) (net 61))
 (segment (start 84 92) (end 82 90) (width 2) (layer F.Cu) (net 61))
 (segment (start 90 92) (end 84 92) (width 2) (layer F.Cu) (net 61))
 (segment (start 76.38 78.38) (end 82 84) (width 2) (layer F.Cu) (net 58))
 (segment (start 76.38 76.89) (end 76.38 78.38) (width 2) (layer F.Cu) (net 58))
 (segment (start 103 92) (end 101 90) (width 2) (layer F.Cu) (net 55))
 (segment (start 109 92) (end 103 92) (width 2) (layer F.Cu) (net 55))
 (segment (start 109 83) (end 109 92) (width 2) (layer F.Cu) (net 55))
 (segment (start 108.08 82.08) (end 109 83) (width 2) (layer F.Cu) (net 55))
 (segment (start 108.08 76.89) (end 108.08 82.08) (width 2) (layer F.Cu) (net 55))
 (segment (start 95.38 78.38) (end 101 84) (width 2) (layer F.Cu) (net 52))
 (segment (start 95.38 76.89) (end 95.38 78.38) (width 2) (layer F.Cu) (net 52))
 (segment (start 107.84 25.84) (end 107 25) (width 1) (layer F.Cu) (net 14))
 (segment (start 107.84 34.38) (end 107.84 25.84) (width 1) (layer F.Cu) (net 14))
 (segment (start 105.3 25.3) (end 105 25) (width 1) (layer F.Cu) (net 15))
 (segment (start 105.3 34.38) (end 105.3 25.3) (width 1) (layer F.Cu) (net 15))
 (segment (start 102.76 25.24) (end 103 25) (width 1) (layer F.Cu) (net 16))
 (segment (start 102.76 34.38) (end 102.76 25.24) (width 1) (layer F.Cu) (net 16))
 (segment (start 100.22 25.78) (end 101 25) (width 1) (layer F.Cu) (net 17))
 (segment (start 100.22 34.38) (end 100.22 25.78) (width 1) (layer F.Cu) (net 17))
 (segment (start 61.62 33.295) (end 65.57 29.345) (width 0.25) (layer F.Cu) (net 41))
 (segment (start 61.62 36.11) (end 61.62 33.295) (width 0.25) (layer F.Cu) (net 41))
 (segment (start 48.92 36.11) (end 48.92 34.08) (width 0.25) (layer F.Cu) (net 42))
 (segment (start 48.92 34.08) (end 56 27) (width 0.25) (layer F.Cu) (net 42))
 (segment (start 56 27) (end 70 27) (width 0.25) (layer F.Cu) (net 42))
 (segment (start 70 27) (end 71 28) (width 0.25) (layer F.Cu) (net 42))
 (segment (start 71 28.995) (end 68.11 31.885) (width 0.25) (layer F.Cu) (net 42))
 (segment (start 71 28) (end 71 28.995) (width 0.25) (layer F.Cu) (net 42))
 (via (at 117 51) (size 0.8) (drill 0.4) (layers F.Cu B.Cu) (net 1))
 (segment (start 97.347 51) (end 117 51) (width 0.25) (layer F.Cu) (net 1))
 (segment (start 88.43 42.083) (end 97.347 51) (width 0.25) (layer F.Cu) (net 1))
 (segment (start 137.232999 48.532999) (end 138.32 49.62) (width 0.25) (layer B.Cu) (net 1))
 (segment (start 135.258239 48.532999) (end 137.232999 48.532999) (width 0.25) (layer B.Cu) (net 1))
 (segment (start 134.692999 49.098239) (end 135.258239 48.532999) (width 0.25) (layer B.Cu) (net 1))
 (segment (start 134.692999 49.775763) (end 134.692999 49.098239) (width 0.25) (layer B.Cu) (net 1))
 (segment (start 133.468762 51) (end 134.692999 49.775763) (width 0.25) (layer B.Cu) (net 1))
 (segment (start 117 51) (end 133.468762 51) (width 0.25) (layer B.Cu) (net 1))
 (segment (start 63 42.075) (end 65.57 39.505) (width 0.25) (layer B.Cu) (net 10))
 (segment (start 63 49) (end 63 42.075) (width 0.25) (layer B.Cu) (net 10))
 (segment (start 64 50) (end 63 49) (width 0.25) (layer B.Cu) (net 10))
 (segment (start 91 50) (end 64 50) (width 0.25) (layer B.Cu) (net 10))
 (segment (start 94 47) (end 91 50) (width 0.25) (layer B.Cu) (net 10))
 (segment (start 115.54 47) (end 94 47) (width 0.25) (layer B.Cu) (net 10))
 (segment (start 128.16 34.38) (end 115.54 47) (width 0.25) (layer B.Cu) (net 10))
 (segment (start 114.372999 50.707001) (end 115.46 49.62) (width 0.25) (layer B.Cu) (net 4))
 (segment (start 64.070591 50.707001) (end 114.372999 50.707001) (width 0.25) (layer B.Cu) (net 4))
 (segment (start 62.549991 49.186401) (end 64.070591 50.707001) (width 0.25) (layer B.Cu) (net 4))
 (segment (start 62.549991 40.004009) (end 62.549991 49.186401) (width 0.25) (layer B.Cu) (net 4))
 (segment (start 65.57 36.984) (end 62.549991 40.004009) (width 0.25) (layer B.Cu) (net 4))
 (segment (start 67.022999 33.337999) (end 77.662001 33.337999) (width 0.25) (layer F.Cu) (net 3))
 (segment (start 65.57 31.885) (end 67.022999 33.337999) (width 0.25) (layer F.Cu) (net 3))
 (segment (start 79.874003 35.550001) (end 93.550001 35.550001) (width 0.25) (layer F.Cu) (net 3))
 (segment (start 77.662001 33.337999) (end 79.874003 35.550001) (width 0.25) (layer F.Cu) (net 3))
 (segment (start 93.550001 35.550001) (end 102 44) (width 0.25) (layer F.Cu) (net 3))
 (via (at 126 44) (size 0.8) (drill 0.4) (layers F.Cu B.Cu) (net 3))
 (segment (start 102 44) (end 126 44) (width 0.25) (layer F.Cu) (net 3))
 (segment (start 127.62 44) (end 133.24 49.62) (width 0.25) (layer B.Cu) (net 3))
 (segment (start 126 44) (end 127.62 44) (width 0.25) (layer B.Cu) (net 3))
 (segment (start 68.11 36.965) (end 71.965 36.965) (width 0.25) (layer F.Cu) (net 2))
 (segment (start 71.965 36.965) (end 87 52) (width 0.25) (layer F.Cu) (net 2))
 (via (at 117 52) (size 0.8) (drill 0.4) (layers F.Cu B.Cu) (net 2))
 (segment (start 87 52) (end 117 52) (width 0.25) (layer F.Cu) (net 2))
 (segment (start 133.4 52) (end 135.78 49.62) (width 0.25) (layer B.Cu) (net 2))
 (segment (start 117 52) (end 133.4 52) (width 0.25) (layer B.Cu) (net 2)))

